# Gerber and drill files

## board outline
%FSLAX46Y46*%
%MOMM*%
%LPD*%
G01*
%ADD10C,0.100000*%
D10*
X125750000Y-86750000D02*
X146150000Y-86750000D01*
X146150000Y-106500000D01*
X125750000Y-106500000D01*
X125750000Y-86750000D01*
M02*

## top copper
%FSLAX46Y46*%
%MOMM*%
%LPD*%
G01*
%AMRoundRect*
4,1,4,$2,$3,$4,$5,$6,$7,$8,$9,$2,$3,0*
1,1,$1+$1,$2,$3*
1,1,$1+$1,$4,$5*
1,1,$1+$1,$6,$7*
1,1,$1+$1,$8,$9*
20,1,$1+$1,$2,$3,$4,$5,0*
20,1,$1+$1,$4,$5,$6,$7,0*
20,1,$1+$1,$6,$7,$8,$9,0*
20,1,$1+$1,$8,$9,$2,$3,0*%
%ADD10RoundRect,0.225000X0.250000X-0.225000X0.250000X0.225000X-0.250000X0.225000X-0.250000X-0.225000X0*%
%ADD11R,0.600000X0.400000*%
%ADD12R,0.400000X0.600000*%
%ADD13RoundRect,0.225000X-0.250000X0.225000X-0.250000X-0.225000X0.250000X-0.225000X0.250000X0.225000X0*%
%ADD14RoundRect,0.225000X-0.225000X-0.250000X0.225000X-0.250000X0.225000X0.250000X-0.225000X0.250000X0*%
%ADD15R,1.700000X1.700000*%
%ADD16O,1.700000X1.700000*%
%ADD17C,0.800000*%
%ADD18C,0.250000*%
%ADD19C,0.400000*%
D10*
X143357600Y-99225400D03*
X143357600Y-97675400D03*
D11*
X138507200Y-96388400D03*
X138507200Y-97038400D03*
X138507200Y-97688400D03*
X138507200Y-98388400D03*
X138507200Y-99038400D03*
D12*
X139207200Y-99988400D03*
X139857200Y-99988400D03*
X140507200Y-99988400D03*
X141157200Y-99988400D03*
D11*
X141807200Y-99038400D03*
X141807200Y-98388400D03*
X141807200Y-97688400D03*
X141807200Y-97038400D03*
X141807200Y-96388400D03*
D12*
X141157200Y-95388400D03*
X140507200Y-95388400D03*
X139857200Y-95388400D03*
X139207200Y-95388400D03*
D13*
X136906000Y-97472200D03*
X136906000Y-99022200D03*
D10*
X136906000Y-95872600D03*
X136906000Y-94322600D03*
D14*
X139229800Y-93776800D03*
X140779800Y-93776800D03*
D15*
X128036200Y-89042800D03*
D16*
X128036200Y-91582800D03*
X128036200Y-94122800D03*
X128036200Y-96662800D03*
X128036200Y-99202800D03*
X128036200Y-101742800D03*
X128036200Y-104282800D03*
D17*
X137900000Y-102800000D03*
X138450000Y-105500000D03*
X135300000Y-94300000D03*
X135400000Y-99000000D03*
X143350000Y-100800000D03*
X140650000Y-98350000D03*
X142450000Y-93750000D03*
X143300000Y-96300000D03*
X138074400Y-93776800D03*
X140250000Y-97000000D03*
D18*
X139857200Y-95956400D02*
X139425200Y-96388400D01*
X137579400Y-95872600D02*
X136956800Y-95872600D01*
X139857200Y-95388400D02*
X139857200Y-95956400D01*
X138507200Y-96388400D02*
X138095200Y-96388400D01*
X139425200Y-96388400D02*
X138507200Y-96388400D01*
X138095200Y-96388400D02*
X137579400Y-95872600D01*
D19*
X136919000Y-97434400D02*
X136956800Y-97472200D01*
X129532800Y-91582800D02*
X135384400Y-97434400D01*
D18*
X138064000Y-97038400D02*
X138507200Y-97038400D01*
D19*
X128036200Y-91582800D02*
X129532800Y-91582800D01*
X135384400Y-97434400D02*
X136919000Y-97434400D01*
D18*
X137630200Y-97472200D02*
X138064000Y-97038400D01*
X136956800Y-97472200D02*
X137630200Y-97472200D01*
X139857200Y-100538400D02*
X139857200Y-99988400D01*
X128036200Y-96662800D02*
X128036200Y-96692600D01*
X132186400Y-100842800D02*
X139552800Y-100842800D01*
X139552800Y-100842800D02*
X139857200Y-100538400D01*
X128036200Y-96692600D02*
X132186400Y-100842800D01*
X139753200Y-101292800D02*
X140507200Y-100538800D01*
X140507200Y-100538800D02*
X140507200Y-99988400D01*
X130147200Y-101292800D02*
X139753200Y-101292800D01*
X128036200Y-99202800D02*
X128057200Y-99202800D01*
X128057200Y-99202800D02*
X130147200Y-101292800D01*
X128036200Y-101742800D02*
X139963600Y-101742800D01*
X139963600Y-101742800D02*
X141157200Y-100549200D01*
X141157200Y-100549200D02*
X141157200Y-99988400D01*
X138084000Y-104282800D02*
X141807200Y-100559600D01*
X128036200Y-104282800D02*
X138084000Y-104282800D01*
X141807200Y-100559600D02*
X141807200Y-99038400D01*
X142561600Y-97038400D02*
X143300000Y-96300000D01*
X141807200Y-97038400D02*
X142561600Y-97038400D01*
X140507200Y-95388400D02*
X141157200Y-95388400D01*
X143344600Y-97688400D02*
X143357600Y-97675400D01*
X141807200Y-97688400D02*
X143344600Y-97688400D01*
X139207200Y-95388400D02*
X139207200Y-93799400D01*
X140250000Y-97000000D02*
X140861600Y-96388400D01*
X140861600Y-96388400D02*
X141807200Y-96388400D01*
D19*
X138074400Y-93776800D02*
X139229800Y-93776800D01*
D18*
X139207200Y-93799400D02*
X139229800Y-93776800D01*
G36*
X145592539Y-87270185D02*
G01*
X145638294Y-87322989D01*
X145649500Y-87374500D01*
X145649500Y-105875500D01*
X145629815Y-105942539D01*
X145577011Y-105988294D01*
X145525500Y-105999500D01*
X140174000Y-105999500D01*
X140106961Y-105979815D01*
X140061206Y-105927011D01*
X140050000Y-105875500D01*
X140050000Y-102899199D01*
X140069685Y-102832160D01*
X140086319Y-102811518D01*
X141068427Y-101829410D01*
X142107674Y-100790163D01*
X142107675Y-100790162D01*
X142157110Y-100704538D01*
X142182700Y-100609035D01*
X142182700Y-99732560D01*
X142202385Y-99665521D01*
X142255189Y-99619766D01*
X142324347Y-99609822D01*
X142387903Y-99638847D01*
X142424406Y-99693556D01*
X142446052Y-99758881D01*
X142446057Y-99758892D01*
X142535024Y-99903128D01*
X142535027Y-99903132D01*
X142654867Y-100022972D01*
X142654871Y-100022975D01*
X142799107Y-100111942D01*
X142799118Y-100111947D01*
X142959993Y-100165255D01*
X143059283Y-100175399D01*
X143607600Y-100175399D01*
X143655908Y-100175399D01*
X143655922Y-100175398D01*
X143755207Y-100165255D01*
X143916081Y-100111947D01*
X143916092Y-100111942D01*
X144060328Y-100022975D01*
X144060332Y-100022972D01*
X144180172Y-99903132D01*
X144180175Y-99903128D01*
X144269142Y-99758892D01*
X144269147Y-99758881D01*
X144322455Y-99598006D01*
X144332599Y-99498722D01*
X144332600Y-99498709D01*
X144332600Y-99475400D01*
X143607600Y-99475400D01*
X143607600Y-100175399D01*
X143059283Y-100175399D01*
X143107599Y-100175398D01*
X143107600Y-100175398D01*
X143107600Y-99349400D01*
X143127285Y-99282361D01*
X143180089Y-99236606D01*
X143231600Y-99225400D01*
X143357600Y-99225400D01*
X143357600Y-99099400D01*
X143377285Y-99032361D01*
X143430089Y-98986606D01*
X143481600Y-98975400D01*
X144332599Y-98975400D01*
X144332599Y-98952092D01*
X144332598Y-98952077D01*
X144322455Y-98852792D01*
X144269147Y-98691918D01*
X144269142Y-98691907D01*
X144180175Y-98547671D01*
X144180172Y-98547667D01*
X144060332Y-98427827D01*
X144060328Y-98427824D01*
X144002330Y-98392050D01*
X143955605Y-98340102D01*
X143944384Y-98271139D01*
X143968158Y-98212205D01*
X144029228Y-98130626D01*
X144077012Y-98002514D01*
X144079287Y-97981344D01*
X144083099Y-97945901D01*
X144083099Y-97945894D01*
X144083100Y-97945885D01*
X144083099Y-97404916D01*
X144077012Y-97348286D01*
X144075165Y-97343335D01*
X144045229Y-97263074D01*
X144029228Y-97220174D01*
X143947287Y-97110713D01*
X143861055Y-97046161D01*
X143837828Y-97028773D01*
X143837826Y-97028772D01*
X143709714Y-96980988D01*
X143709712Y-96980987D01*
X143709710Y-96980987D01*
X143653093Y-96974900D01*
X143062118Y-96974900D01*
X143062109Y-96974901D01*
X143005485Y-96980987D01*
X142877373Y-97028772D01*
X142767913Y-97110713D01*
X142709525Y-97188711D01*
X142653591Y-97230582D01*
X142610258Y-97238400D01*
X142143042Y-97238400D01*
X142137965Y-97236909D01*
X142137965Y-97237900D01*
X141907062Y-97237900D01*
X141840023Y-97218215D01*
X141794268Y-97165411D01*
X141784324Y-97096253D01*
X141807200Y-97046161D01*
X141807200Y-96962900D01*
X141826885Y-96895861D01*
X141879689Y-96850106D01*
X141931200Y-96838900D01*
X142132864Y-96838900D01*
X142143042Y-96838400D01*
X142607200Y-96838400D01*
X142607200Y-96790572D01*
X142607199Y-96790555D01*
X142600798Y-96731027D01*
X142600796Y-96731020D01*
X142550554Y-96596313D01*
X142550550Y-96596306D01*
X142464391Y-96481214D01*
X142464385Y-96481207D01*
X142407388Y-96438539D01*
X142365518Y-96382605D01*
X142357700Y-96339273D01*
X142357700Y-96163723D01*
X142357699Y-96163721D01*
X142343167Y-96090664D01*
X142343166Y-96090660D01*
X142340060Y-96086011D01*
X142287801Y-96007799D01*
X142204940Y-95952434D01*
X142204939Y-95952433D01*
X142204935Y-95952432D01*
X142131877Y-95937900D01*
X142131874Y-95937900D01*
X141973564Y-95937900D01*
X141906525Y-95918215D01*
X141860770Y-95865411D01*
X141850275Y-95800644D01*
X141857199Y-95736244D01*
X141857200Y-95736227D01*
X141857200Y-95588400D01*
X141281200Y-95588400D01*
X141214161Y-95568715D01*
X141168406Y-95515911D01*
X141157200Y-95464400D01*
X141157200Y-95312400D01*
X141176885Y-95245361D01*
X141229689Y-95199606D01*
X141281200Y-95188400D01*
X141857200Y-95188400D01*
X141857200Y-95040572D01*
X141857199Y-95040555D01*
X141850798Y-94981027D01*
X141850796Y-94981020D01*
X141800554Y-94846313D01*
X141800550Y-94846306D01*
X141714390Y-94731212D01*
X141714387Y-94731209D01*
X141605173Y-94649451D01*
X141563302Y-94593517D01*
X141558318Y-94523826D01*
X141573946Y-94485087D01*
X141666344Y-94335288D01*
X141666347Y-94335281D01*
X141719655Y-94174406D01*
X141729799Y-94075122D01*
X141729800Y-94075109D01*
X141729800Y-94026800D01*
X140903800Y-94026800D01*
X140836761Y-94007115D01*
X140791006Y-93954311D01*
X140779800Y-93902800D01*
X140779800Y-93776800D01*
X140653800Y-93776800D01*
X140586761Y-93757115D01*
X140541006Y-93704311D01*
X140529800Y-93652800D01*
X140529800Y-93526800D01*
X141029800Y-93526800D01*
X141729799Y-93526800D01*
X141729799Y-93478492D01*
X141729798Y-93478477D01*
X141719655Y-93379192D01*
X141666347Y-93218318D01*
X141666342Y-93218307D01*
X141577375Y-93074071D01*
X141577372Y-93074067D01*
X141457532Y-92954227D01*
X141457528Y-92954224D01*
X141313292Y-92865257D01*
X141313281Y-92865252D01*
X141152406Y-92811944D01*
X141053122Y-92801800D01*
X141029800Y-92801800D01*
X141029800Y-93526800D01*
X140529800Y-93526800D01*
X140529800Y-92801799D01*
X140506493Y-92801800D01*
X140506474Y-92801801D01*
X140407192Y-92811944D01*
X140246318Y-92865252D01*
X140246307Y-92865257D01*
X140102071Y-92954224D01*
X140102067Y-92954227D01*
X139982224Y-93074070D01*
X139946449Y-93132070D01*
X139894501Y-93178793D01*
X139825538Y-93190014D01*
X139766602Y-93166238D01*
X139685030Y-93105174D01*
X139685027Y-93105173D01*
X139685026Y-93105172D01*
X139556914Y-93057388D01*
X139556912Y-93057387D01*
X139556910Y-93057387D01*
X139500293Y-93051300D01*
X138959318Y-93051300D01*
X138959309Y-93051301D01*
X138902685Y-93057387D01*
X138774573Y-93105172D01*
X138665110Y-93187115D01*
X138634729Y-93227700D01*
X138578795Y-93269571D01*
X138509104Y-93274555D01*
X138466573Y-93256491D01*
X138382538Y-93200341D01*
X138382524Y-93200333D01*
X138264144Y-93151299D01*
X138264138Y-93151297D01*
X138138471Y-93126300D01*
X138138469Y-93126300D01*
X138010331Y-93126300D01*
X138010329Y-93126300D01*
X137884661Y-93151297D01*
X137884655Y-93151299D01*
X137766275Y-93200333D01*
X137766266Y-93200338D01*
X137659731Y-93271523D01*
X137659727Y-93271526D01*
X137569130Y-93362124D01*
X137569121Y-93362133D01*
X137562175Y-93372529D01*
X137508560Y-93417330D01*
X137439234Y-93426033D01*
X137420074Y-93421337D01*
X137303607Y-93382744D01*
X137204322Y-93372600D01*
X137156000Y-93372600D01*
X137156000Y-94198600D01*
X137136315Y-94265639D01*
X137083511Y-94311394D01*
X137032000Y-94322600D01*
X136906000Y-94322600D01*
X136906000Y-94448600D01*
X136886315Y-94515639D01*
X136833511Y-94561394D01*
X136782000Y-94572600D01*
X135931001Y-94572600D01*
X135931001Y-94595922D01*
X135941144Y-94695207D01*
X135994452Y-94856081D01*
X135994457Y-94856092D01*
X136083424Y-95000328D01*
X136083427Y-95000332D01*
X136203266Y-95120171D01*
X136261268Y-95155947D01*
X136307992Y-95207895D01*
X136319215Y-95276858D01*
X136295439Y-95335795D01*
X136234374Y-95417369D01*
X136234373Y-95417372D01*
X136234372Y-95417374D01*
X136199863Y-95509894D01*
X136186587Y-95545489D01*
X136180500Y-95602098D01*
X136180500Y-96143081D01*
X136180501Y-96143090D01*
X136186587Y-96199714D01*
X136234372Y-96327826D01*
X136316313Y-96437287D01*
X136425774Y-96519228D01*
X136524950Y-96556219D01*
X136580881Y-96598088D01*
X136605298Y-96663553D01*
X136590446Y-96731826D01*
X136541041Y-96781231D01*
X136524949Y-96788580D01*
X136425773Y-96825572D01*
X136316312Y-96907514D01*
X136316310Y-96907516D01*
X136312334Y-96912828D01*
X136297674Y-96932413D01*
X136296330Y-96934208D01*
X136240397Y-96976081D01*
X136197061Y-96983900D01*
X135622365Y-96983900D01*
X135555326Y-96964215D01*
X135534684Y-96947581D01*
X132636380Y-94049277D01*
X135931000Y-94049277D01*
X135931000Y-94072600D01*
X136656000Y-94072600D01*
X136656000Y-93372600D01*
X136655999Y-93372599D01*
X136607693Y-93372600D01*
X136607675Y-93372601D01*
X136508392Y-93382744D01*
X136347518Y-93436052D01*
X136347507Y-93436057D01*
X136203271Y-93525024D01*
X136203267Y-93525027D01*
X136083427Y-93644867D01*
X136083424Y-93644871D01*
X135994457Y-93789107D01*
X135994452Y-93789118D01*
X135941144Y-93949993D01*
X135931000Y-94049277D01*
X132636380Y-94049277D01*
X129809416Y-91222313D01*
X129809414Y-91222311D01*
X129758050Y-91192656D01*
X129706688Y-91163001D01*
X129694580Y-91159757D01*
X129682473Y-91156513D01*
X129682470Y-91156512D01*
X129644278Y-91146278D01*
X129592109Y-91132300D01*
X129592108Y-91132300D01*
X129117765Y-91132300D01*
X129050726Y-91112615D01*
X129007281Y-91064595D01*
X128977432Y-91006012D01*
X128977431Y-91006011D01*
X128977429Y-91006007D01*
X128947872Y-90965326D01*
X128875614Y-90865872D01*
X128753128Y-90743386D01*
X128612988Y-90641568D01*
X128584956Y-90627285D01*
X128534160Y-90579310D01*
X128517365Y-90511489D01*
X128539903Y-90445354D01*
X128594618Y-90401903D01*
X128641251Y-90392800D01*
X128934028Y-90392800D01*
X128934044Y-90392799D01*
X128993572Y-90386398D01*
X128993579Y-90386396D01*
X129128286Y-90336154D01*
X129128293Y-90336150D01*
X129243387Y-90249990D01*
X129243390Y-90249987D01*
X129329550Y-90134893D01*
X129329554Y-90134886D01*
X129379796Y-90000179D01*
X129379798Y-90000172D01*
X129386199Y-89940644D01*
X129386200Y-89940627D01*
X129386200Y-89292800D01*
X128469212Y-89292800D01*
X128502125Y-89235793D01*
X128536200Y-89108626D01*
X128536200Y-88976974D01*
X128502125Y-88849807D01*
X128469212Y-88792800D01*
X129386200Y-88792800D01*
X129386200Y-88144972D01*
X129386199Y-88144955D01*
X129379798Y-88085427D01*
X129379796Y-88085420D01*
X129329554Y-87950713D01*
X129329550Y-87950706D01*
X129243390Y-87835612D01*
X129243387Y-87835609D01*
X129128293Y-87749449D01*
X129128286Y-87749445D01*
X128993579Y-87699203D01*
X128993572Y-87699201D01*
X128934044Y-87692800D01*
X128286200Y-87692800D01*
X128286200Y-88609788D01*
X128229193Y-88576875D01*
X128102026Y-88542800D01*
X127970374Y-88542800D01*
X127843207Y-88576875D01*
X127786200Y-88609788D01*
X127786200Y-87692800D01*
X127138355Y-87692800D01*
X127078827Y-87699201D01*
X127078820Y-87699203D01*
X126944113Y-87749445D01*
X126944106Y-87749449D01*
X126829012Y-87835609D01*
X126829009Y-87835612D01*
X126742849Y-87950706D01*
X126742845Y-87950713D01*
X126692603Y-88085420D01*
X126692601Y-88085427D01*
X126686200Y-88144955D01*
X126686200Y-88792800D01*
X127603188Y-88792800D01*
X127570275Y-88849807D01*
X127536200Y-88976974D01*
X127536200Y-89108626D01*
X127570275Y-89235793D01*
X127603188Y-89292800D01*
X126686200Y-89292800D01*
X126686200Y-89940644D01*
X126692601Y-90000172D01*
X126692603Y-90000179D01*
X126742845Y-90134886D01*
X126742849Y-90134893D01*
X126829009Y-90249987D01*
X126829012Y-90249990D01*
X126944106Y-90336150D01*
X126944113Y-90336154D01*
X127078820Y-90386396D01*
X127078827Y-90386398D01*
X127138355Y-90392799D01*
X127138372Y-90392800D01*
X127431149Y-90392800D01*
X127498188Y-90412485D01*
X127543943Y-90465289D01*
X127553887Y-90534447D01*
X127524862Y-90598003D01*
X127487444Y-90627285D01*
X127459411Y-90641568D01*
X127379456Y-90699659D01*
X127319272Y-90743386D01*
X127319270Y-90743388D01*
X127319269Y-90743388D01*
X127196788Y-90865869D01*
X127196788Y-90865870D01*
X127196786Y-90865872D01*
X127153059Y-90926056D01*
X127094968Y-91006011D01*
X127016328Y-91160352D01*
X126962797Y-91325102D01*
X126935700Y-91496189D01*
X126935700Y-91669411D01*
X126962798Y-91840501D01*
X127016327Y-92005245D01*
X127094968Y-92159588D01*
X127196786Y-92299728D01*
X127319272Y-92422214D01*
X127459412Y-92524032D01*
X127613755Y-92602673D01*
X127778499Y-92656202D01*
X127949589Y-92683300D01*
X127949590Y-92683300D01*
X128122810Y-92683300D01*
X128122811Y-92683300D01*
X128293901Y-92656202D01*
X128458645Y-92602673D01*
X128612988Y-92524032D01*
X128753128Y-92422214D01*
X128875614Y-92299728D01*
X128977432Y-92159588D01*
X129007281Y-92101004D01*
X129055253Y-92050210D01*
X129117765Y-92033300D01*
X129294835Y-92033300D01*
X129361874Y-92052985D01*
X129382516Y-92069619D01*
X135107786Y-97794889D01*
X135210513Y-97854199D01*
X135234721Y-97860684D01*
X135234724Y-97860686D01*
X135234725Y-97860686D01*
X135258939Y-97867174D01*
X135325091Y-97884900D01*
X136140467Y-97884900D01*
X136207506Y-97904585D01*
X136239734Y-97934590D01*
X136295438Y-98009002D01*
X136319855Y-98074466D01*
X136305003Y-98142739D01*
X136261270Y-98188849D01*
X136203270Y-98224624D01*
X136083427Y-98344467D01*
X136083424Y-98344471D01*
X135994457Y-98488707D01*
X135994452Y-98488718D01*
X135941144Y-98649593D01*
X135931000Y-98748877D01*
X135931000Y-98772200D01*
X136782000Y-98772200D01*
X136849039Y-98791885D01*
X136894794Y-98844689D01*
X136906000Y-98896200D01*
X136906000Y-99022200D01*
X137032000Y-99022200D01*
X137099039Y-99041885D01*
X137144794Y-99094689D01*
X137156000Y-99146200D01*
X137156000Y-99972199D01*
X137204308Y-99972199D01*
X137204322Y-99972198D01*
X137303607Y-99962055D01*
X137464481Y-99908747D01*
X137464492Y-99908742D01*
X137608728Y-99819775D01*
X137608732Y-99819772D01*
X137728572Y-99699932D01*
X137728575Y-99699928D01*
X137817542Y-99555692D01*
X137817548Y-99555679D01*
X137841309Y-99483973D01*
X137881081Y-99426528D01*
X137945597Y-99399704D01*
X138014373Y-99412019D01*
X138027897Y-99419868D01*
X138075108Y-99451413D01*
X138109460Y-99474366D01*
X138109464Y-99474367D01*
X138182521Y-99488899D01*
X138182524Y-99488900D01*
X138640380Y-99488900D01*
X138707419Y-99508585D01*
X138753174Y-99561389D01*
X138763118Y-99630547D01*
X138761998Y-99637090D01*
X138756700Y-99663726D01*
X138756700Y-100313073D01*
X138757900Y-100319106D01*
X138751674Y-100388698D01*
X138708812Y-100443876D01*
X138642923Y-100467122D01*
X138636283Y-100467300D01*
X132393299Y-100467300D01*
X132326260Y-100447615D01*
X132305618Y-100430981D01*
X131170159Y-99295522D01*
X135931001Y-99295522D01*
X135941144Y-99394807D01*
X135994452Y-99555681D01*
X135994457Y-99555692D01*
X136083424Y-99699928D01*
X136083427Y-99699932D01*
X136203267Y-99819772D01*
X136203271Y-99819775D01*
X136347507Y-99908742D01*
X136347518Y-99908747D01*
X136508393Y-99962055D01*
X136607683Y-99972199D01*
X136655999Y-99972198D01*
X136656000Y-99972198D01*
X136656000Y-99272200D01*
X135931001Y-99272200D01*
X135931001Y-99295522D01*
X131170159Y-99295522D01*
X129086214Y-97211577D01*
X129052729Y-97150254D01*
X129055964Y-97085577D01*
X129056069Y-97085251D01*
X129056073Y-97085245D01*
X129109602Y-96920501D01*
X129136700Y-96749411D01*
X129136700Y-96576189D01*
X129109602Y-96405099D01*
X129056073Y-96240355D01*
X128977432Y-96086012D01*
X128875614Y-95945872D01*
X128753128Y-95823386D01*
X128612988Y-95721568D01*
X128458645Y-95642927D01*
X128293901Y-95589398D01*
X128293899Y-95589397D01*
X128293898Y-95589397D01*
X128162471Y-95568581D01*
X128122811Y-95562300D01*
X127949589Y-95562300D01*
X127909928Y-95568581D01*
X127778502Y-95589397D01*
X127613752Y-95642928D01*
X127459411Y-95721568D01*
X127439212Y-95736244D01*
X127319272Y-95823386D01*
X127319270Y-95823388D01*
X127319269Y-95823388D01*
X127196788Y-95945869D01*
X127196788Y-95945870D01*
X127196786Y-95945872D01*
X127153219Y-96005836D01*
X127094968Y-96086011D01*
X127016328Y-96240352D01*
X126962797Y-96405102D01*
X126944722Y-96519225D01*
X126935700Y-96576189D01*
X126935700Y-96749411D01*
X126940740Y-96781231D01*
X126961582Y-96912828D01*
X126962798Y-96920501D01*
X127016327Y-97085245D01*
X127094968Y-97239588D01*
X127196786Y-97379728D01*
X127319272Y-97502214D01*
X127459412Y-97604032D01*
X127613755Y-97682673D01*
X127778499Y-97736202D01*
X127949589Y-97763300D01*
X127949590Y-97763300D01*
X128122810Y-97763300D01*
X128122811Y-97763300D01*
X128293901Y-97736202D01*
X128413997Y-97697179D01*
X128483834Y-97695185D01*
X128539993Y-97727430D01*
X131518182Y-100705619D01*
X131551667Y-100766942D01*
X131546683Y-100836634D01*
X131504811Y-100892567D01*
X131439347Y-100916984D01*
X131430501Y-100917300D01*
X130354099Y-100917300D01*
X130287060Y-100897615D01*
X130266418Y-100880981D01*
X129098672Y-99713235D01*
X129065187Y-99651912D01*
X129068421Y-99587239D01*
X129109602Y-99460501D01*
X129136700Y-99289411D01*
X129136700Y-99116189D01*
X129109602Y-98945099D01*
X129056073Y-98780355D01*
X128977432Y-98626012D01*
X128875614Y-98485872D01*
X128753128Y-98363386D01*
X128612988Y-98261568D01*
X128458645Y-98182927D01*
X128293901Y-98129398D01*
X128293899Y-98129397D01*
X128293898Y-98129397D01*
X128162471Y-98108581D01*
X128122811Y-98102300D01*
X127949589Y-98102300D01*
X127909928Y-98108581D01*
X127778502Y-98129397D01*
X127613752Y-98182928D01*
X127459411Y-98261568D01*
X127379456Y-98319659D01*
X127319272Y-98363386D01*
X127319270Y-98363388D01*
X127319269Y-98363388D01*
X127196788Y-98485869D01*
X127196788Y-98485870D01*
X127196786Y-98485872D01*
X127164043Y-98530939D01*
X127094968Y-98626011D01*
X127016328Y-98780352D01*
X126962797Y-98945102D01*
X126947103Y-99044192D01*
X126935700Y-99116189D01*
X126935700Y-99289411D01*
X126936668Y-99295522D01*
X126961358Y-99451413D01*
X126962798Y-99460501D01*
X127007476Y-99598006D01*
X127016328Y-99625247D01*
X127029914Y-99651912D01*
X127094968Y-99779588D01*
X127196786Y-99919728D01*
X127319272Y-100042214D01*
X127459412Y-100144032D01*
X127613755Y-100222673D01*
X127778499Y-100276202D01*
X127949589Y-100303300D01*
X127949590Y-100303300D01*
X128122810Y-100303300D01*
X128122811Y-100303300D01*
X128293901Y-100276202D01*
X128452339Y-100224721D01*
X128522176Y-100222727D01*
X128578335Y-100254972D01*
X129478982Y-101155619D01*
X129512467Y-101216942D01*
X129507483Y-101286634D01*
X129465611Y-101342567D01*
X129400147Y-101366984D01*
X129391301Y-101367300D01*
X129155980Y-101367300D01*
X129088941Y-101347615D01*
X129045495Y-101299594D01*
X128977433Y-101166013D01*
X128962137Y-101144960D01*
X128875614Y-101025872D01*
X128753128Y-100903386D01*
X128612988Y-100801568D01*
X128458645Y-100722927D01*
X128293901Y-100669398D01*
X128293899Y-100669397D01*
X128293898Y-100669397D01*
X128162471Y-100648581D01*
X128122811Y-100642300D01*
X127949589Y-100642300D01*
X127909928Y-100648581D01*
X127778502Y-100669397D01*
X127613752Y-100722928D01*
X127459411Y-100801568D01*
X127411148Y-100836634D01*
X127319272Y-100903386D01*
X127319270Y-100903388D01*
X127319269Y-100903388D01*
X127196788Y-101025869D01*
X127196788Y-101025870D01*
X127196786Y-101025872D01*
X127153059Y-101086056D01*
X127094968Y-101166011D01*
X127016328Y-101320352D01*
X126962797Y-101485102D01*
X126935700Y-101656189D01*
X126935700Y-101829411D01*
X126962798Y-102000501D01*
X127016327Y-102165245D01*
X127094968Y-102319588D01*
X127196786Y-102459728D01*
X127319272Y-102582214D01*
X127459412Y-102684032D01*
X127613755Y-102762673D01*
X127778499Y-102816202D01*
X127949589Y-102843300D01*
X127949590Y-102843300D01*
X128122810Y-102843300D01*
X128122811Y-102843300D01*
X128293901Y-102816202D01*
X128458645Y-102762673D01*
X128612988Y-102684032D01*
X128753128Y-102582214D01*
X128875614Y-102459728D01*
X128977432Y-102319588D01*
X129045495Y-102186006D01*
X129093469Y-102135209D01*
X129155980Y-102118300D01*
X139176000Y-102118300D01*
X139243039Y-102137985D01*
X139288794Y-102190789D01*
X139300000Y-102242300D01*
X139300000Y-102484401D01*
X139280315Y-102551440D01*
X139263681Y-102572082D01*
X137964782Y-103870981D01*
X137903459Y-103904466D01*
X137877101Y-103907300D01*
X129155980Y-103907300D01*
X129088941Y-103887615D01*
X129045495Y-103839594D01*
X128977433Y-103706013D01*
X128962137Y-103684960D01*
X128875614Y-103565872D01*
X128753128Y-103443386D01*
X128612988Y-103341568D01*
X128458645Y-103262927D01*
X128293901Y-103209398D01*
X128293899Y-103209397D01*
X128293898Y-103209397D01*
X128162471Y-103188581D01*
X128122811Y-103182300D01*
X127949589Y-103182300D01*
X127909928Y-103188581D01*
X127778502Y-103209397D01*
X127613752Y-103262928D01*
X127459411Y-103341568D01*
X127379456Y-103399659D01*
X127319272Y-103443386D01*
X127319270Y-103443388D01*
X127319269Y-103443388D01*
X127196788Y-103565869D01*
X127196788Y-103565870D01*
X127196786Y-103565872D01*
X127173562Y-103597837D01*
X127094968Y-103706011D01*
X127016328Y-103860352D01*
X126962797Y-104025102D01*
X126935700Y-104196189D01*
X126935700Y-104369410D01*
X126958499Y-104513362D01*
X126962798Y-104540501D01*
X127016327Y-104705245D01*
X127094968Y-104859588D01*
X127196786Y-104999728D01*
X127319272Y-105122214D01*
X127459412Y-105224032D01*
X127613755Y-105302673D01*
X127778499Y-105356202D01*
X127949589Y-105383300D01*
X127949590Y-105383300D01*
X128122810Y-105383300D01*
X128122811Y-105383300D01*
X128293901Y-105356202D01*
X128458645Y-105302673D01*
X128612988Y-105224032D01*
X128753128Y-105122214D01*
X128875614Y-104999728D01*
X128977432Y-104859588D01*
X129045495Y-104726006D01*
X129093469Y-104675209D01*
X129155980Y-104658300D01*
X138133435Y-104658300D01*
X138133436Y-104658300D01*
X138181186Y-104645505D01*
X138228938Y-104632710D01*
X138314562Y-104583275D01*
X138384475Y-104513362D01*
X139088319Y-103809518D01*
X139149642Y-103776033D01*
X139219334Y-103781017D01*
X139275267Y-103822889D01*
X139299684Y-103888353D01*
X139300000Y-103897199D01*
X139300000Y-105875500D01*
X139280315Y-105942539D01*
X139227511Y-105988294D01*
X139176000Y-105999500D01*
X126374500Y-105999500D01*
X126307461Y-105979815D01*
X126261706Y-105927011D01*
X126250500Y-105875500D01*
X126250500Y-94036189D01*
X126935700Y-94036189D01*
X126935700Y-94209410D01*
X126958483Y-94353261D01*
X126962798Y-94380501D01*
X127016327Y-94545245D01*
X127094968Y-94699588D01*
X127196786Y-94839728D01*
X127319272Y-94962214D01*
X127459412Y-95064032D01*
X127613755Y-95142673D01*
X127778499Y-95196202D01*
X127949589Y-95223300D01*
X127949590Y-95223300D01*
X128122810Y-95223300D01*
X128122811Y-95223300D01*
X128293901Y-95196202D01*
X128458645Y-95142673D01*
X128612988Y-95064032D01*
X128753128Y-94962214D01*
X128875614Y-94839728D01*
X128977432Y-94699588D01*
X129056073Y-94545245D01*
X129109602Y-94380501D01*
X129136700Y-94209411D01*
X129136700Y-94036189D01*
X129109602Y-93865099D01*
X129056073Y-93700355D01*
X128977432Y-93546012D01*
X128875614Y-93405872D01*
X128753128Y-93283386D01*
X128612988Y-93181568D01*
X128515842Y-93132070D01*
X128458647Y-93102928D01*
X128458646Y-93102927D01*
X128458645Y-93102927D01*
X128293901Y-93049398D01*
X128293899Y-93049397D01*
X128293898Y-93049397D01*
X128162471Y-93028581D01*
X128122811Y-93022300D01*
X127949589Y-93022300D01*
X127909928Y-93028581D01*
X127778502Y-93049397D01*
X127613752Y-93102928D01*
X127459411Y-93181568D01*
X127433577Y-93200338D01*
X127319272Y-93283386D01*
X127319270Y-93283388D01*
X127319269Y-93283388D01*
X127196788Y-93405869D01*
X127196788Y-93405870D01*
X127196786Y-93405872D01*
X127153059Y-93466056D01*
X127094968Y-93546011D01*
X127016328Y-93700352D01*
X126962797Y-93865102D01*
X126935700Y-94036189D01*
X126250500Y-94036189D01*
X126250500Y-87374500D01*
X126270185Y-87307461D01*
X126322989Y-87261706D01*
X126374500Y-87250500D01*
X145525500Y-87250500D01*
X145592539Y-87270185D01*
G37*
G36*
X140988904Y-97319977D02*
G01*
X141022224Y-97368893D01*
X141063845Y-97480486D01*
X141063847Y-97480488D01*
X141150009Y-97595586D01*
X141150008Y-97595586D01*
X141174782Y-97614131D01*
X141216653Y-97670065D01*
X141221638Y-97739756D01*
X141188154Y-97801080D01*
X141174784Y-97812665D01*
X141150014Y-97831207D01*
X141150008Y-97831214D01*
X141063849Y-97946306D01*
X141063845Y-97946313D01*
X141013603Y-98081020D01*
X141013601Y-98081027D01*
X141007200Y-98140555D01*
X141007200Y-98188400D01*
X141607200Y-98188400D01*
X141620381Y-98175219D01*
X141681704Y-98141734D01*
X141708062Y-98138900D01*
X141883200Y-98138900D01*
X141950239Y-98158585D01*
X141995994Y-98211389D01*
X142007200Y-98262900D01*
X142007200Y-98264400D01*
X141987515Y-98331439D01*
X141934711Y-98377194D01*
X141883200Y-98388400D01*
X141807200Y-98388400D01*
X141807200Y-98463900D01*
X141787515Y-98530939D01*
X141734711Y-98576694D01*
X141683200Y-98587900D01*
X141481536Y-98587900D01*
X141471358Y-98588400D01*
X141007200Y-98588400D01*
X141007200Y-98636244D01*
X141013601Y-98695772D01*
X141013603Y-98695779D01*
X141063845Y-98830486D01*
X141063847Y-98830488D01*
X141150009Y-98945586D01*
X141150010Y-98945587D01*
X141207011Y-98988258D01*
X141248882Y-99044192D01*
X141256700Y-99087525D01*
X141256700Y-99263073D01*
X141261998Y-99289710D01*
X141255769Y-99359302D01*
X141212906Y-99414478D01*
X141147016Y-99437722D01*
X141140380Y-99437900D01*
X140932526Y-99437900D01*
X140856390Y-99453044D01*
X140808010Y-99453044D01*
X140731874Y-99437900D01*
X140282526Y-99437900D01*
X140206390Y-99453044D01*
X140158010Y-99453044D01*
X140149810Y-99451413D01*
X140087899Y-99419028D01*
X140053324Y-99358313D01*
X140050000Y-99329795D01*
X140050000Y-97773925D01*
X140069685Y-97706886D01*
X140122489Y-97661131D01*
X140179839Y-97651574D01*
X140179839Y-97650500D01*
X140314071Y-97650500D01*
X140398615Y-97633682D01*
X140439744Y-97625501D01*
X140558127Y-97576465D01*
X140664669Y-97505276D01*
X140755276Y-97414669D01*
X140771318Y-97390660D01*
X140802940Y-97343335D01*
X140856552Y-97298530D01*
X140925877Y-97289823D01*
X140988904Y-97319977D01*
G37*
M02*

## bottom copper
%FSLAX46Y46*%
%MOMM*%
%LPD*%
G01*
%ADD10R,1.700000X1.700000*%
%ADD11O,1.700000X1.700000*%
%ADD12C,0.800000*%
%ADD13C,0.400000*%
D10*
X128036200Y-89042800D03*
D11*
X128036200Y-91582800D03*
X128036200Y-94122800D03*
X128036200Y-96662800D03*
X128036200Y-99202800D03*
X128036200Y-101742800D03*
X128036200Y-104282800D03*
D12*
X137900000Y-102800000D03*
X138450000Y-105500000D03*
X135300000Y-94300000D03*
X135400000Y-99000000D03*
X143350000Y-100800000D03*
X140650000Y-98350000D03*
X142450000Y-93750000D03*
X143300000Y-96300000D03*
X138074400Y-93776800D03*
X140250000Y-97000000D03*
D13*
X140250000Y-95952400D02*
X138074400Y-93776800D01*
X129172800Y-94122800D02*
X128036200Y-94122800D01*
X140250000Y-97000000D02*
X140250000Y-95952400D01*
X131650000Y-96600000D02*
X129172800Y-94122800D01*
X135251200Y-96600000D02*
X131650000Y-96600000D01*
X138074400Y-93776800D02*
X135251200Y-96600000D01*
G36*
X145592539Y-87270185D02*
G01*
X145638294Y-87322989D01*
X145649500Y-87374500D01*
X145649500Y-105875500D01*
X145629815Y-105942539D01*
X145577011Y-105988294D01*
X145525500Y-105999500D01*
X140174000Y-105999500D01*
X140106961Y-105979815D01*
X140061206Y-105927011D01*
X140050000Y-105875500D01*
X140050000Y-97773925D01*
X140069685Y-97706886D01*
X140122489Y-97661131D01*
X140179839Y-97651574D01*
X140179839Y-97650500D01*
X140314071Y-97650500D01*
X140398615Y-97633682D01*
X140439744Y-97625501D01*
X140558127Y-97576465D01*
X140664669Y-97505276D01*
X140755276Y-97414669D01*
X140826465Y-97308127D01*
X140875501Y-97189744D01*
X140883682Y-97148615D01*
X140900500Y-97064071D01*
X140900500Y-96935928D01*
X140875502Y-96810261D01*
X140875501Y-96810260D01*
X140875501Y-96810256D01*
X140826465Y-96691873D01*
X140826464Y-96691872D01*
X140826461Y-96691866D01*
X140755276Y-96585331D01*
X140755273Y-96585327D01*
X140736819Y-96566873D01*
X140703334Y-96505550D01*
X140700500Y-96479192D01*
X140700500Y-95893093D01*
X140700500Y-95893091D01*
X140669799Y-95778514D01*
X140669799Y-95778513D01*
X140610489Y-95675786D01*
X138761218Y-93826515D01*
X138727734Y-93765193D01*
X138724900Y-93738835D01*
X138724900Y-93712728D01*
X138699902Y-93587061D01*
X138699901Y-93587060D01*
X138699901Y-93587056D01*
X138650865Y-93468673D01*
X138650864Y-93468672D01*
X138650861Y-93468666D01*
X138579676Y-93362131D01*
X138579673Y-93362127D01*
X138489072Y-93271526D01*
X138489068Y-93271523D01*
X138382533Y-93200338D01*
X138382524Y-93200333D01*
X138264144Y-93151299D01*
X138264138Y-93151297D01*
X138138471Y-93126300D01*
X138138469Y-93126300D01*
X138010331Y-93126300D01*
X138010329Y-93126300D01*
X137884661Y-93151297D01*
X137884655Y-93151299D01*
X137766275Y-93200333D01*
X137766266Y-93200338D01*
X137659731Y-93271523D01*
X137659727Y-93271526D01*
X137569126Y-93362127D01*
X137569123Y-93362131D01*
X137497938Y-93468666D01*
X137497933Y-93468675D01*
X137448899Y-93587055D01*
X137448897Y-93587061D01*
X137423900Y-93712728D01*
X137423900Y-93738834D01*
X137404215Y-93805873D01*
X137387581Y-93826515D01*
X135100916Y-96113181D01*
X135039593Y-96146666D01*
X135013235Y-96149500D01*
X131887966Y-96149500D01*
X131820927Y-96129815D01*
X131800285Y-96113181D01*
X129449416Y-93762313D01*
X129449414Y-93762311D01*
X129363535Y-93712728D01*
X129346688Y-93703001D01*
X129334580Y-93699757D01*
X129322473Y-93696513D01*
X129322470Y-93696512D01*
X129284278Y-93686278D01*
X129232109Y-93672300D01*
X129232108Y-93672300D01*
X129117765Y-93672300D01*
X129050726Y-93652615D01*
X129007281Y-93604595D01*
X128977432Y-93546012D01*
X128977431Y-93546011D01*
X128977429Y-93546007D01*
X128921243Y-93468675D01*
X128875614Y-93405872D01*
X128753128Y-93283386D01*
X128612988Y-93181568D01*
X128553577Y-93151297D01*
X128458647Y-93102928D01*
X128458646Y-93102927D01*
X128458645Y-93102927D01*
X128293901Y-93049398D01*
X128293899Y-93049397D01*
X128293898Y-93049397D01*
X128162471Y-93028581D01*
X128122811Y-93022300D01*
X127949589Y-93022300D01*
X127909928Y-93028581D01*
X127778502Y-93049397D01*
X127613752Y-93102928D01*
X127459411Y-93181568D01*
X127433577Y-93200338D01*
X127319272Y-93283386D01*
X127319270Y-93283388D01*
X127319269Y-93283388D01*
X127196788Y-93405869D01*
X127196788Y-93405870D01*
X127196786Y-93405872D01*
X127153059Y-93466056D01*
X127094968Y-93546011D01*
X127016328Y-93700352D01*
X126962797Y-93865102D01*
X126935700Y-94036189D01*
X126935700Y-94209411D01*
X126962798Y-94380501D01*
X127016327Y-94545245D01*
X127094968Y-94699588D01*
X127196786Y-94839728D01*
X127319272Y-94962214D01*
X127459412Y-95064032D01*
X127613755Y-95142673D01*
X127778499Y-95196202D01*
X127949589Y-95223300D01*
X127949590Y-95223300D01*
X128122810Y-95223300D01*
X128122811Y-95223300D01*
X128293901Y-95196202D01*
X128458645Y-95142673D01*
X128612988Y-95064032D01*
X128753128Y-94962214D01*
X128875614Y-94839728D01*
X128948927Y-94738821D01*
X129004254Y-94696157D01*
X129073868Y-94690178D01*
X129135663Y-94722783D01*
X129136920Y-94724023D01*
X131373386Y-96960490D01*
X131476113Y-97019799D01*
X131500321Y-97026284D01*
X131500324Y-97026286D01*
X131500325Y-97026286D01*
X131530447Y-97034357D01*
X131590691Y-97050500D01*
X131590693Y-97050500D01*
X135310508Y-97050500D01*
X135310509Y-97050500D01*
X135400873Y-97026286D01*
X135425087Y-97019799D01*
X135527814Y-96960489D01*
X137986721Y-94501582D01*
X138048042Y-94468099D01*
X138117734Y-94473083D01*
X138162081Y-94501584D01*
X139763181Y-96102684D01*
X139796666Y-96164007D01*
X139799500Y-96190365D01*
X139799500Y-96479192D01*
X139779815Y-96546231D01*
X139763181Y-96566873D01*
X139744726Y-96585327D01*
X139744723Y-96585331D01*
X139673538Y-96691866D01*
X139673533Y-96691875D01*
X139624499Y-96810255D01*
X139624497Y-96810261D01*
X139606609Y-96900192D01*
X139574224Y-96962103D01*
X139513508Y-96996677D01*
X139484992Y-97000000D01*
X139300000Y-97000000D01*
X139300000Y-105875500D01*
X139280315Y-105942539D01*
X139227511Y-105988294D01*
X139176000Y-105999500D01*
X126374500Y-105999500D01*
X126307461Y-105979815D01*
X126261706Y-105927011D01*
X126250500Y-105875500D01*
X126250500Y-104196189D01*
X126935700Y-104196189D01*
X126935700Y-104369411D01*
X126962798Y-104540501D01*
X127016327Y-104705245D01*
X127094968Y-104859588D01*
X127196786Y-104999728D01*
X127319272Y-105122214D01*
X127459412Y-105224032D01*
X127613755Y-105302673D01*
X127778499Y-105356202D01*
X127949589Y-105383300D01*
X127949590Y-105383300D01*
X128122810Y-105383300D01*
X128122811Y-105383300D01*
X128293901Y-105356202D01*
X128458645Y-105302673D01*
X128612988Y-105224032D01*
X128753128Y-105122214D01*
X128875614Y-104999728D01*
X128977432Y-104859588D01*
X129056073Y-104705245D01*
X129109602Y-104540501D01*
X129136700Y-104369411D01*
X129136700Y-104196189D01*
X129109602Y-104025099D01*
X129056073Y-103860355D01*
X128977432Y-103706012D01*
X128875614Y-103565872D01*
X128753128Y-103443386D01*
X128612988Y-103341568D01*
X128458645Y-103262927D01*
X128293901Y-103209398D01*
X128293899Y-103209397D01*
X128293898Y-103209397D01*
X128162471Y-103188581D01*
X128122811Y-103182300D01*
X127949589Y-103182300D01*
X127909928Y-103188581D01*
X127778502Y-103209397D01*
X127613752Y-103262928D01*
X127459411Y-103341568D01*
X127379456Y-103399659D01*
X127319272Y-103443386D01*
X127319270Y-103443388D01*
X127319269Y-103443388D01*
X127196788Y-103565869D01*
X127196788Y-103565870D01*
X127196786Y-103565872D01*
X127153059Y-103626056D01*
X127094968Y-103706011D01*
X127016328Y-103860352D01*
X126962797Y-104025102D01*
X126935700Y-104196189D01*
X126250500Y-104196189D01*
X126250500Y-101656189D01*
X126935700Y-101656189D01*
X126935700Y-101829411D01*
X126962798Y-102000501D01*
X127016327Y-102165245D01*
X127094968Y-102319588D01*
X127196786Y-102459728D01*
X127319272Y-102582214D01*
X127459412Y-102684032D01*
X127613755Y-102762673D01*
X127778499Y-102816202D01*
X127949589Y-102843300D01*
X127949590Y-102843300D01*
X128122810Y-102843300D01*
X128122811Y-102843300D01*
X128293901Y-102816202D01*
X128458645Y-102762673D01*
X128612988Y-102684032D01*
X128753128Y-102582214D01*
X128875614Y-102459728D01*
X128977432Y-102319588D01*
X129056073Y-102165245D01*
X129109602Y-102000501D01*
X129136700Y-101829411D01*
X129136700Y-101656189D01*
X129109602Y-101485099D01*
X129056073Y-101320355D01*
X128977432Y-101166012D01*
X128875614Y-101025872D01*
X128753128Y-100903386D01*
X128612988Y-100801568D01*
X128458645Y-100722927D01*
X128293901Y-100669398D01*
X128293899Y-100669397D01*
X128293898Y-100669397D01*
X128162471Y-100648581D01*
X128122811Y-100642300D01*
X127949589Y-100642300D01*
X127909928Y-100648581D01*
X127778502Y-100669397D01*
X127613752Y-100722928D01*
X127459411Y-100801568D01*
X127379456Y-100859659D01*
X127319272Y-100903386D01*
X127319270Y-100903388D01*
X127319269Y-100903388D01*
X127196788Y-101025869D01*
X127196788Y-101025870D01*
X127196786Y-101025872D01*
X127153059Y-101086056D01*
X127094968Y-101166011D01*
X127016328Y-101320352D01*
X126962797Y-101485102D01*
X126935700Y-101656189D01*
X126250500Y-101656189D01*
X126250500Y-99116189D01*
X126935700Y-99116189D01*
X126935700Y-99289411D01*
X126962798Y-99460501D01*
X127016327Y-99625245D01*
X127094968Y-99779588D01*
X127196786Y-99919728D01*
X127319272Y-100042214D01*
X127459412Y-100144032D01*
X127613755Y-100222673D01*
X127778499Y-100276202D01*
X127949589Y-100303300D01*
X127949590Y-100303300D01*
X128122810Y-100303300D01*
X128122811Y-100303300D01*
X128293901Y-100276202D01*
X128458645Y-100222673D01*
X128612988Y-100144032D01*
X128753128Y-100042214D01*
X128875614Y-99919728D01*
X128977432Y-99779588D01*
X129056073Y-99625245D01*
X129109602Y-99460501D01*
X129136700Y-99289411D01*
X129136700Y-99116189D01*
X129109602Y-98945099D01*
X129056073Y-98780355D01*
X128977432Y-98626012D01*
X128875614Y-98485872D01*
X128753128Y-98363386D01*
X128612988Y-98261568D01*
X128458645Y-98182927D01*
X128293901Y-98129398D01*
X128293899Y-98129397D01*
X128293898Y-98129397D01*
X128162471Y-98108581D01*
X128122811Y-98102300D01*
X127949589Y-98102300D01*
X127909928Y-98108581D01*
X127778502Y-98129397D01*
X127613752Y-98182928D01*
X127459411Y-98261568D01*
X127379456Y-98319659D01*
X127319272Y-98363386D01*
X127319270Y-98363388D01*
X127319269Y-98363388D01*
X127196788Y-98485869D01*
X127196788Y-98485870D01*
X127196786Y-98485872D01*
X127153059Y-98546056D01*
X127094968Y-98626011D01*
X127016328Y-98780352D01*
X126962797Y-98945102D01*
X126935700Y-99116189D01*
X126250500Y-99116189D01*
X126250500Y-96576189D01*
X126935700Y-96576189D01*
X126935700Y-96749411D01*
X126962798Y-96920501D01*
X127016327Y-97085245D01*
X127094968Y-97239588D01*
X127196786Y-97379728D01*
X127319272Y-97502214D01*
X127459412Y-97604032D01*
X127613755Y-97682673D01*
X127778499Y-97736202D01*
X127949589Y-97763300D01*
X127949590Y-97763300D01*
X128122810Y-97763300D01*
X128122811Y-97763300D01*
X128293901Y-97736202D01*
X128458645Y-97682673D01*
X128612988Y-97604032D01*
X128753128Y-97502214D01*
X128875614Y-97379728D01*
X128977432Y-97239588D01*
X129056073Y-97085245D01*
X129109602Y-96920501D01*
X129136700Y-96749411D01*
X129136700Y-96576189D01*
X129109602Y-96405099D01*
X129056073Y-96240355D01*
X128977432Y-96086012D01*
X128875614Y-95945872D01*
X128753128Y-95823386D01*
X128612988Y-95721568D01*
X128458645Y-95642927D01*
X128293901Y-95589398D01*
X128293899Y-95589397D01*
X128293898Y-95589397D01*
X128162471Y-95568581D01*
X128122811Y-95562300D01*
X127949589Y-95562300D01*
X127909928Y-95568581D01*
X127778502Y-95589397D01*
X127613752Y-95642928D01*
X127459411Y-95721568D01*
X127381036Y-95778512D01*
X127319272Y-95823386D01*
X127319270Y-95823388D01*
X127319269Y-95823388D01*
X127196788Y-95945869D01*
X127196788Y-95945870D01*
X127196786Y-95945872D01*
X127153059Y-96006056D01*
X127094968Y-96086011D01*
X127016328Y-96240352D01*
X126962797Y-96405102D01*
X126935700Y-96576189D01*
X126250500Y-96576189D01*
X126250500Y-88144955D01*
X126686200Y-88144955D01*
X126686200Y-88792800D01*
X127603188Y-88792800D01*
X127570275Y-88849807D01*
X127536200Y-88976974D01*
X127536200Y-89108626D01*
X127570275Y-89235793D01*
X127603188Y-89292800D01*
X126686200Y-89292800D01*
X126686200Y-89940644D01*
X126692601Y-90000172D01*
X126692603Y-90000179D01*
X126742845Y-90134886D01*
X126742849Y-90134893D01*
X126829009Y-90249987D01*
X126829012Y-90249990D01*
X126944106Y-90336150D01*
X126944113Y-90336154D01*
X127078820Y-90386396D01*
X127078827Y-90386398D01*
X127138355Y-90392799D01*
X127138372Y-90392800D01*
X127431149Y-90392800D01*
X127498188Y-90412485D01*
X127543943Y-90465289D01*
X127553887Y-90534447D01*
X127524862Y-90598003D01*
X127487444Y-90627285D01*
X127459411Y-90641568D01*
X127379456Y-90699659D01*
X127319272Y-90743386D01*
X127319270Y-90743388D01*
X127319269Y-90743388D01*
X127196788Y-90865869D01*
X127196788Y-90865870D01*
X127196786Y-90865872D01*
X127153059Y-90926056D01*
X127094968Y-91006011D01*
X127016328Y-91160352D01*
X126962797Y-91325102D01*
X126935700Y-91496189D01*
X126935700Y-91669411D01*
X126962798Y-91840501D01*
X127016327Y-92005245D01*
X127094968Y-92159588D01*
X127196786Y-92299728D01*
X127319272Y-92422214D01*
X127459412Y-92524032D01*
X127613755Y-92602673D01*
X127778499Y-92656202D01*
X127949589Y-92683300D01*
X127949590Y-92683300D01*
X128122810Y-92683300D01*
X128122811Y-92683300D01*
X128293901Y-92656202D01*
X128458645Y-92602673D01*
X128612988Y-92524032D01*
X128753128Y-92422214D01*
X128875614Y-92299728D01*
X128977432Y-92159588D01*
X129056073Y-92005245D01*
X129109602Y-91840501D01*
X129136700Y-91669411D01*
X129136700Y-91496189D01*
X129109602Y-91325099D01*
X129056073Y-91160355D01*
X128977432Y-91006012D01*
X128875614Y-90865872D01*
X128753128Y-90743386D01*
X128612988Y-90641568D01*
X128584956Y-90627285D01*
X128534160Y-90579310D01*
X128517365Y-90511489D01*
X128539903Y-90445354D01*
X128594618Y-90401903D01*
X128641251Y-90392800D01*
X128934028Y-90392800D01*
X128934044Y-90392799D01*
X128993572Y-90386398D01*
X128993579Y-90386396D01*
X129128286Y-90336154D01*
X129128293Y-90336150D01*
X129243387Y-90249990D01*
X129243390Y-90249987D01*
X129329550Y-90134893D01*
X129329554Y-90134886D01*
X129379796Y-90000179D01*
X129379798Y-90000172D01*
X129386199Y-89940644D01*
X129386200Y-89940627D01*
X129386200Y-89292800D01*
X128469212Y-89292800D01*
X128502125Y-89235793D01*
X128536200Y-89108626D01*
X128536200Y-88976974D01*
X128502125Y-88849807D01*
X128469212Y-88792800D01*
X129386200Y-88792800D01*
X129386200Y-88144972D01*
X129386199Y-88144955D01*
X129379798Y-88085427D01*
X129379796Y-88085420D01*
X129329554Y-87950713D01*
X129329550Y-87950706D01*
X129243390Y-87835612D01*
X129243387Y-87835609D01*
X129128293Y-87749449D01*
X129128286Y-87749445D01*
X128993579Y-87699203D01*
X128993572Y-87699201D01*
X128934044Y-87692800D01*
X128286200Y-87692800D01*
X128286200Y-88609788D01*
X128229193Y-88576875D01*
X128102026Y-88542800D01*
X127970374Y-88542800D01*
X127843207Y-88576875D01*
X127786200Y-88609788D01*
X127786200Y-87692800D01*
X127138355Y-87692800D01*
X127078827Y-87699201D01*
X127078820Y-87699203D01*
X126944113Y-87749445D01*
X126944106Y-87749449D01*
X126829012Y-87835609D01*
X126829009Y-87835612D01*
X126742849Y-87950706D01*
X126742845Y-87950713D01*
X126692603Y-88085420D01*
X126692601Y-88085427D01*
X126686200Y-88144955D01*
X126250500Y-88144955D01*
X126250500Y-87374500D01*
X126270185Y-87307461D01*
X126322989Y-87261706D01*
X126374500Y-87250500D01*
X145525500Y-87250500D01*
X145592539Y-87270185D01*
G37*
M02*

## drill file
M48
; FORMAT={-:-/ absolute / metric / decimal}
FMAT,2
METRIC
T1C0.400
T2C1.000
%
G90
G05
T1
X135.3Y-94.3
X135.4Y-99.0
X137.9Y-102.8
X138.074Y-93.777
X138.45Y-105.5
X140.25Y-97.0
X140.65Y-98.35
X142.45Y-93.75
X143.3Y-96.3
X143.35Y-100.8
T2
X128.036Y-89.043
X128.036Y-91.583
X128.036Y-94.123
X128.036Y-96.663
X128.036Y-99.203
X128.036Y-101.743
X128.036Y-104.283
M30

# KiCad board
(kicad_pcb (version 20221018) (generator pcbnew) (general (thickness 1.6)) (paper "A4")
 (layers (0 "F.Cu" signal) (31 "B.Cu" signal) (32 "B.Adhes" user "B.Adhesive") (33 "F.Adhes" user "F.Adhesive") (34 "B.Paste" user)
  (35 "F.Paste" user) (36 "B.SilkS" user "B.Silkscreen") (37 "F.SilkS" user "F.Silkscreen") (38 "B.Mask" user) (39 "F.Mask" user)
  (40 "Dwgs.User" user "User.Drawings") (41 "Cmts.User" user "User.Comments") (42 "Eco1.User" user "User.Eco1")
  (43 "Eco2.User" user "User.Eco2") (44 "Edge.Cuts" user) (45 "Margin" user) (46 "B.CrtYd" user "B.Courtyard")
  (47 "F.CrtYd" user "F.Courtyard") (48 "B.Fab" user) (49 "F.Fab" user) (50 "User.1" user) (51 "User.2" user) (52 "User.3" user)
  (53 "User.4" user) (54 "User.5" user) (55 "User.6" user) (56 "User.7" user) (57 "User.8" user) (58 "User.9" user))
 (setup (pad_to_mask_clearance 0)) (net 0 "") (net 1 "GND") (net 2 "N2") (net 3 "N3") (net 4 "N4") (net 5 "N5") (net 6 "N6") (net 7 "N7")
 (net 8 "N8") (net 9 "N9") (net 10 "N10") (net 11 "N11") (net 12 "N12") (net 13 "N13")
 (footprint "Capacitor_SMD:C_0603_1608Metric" (layer "F.Cu") (at 143.3576 98.4504 90)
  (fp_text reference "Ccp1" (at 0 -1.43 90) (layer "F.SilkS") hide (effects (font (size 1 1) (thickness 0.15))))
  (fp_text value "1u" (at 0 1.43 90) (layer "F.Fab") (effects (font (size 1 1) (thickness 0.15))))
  (pad "1" smd roundrect (at -0.775 0 90) (size 0.9 0.95) (layers "F.Cu" "F.Paste" "F.Mask") (roundrect_rratio 0.25) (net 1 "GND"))
  (pad "2" smd roundrect (at 0.775 0 90) (size 0.9 0.95) (layers "F.Cu" "F.Paste" "F.Mask") (roundrect_rratio 0.25) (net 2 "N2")))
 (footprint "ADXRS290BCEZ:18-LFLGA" (layer "F.Cu") (at 140.1572 97.6884)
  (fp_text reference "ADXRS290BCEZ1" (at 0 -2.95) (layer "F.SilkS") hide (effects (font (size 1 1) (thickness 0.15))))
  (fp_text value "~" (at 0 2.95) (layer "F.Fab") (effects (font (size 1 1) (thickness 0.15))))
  (pad "1" smd rect (at -1.65 -1.3) (size 0.6 0.4) (layers "F.Cu" "F.Paste" "F.Mask") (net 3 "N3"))
  (pad "2" smd rect (at -1.65 -0.65) (size 0.6 0.4) (layers "F.Cu" "F.Paste" "F.Mask") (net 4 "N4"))
  (pad "3" smd rect (at -1.65 0) (size 0.6 0.4) (layers "F.Cu" "F.Paste" "F.Mask") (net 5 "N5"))
  (pad "4" smd rect (at -1.65 0.7) (size 0.6 0.4) (layers "F.Cu" "F.Paste" "F.Mask") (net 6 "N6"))
  (pad "5" smd rect (at -1.65 1.35) (size 0.6 0.4) (layers "F.Cu" "F.Paste" "F.Mask") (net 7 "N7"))
  (pad "6" smd rect (at -0.95 2.3 90) (size 0.6 0.4) (layers "F.Cu" "F.Paste" "F.Mask") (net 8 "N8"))
  (pad "7" smd rect (at -0.3 2.3 90) (size 0.6 0.4) (layers "F.Cu" "F.Paste" "F.Mask") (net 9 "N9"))
  (pad "8" smd rect (at 0.35 2.3 90) (size 0.6 0.4) (layers "F.Cu" "F.Paste" "F.Mask") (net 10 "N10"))
  (pad "9" smd rect (at 1 2.3 90) (size 0.6 0.4) (layers "F.Cu" "F.Paste" "F.Mask") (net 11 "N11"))
  (pad "10" smd rect (at 1.65 1.35 180) (size 0.6 0.4) (layers "F.Cu" "F.Paste" "F.Mask") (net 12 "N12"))
  (pad "11" smd rect (at 1.65 0.7 180) (size 0.6 0.4) (layers "F.Cu" "F.Paste" "F.Mask") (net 1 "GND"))
  (pad "12" smd rect (at 1.65 0 180) (size 0.6 0.4) (layers "F.Cu" "F.Paste" "F.Mask") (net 2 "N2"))
  (pad "13" smd rect (at 1.65 -0.65 180) (size 0.6 0.4) (layers "F.Cu" "F.Paste" "F.Mask") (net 1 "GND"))
  (pad "14" smd rect (at 1.65 -1.3 180) (size 0.6 0.4) (layers "F.Cu" "F.Paste" "F.Mask") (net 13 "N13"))
  (pad "15" smd rect (at 1 -2.3 90) (size 0.6 0.4) (layers "F.Cu" "F.Paste" "F.Mask") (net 1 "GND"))
  (pad "16" smd rect (at 0.35 -2.3 90) (size 0.6 0.4) (layers "F.Cu" "F.Paste" "F.Mask") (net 1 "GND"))
  (pad "17" smd rect (at -0.3 -2.3 90) (size 0.6 0.4) (layers "F.Cu" "F.Paste" "F.Mask") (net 3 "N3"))
  (pad "18" smd rect (at -0.95 -2.3 90) (size 0.6 0.4) (layers "F.Cu" "F.Paste" "F.Mask") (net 13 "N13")))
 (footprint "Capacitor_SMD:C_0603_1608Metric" (layer "F.Cu") (at 136.906 98.2472 -90)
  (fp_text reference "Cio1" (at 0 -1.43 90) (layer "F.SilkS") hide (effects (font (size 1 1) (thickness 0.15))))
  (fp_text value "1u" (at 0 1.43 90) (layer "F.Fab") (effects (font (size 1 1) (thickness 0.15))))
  (pad "1" smd roundrect (at -0.775 0 270) (size 0.9 0.95) (layers "F.Cu" "F.Paste" "F.Mask") (roundrect_rratio 0.25) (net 4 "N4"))
  (pad "2" smd roundrect (at 0.775 0 270) (size 0.9 0.95) (layers "F.Cu" "F.Paste" "F.Mask") (roundrect_rratio 0.25) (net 1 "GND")))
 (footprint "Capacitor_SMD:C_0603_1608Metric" (layer "F.Cu") (at 136.906 95.0976 90)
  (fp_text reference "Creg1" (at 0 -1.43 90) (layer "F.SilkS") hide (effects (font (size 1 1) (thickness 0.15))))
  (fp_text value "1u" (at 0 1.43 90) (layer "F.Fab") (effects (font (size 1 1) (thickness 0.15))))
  (pad "1" smd roundrect (at -0.775 0 90) (size 0.9 0.95) (layers "F.Cu" "F.Paste" "F.Mask") (roundrect_rratio 0.25) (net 3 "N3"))
  (pad "2" smd roundrect (at 0.775 0 90) (size 0.9 0.95) (layers "F.Cu" "F.Paste" "F.Mask") (roundrect_rratio 0.25) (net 1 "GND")))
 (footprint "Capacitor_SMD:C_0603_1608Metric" (layer "F.Cu") (at 140.0048 93.7768)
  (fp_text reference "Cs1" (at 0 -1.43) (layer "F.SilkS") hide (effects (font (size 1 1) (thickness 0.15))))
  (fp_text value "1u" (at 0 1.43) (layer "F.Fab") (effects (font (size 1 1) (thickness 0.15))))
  (pad "1" smd roundrect (at -0.775 0) (size 0.9 0.95) (layers "F.Cu" "F.Paste" "F.Mask") (roundrect_rratio 0.25) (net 13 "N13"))
  (pad "2" smd roundrect (at 0.775 0) (size 0.9 0.95) (layers "F.Cu" "F.Paste" "F.Mask") (roundrect_rratio 0.25) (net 1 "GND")))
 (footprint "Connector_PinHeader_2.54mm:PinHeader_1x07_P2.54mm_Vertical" (layer "F.Cu") (at 128.0362 89.0428)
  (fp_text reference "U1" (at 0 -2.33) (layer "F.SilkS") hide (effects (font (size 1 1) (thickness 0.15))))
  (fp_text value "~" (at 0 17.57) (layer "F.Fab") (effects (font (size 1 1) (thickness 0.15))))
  (pad "1" thru_hole rect (at 0 0) (size 1.7 1.7) (drill 1) (layers "*.Cu" "*.Mask") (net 1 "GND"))
  (pad "2" thru_hole oval (at 0 2.54) (size 1.7 1.7) (drill 1) (layers "*.Cu" "*.Mask") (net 4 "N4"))
  (pad "3" thru_hole oval (at 0 5.08) (size 1.7 1.7) (drill 1) (layers "*.Cu" "*.Mask") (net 13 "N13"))
  (pad "4" thru_hole oval (at 0 7.62) (size 1.7 1.7) (drill 1) (layers "*.Cu" "*.Mask") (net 9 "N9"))
  (pad "5" thru_hole oval (at 0 10.16) (size 1.7 1.7) (drill 1) (layers "*.Cu" "*.Mask") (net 10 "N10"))
  (pad "6" thru_hole oval (at 0 12.7) (size 1.7 1.7) (drill 1) (layers "*.Cu" "*.Mask") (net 11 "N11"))
  (pad "7" thru_hole oval (at 0 15.24) (size 1.7 1.7) (drill 1) (layers "*.Cu" "*.Mask") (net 12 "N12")))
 (gr_rect (start 125.75 86.75) (end 146.15 106.5) (stroke (width 0.1) (type default)) (fill none) (layer "Edge.Cuts"))
 (segment (start 139.8572 95.9564) (end 139.4252 96.3884) (width 0.25) (layer "F.Cu") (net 3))
 (segment (start 137.5794 95.8726) (end 136.9568 95.8726) (width 0.25) (layer "F.Cu") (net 3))
 (segment (start 139.8572 95.3884) (end 139.8572 95.9564) (width 0.25) (layer "F.Cu") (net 3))
 (segment (start 138.5072 96.3884) (end 138.0952 96.3884) (width 0.25) (layer "F.Cu") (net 3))
 (segment (start 139.4252 96.3884) (end 138.5072 96.3884) (width 0.25) (layer "F.Cu") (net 3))
 (segment (start 138.0952 96.3884) (end 137.5794 95.8726) (width 0.25) (layer "F.Cu") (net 3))
 (segment (start 136.919 97.4344) (end 136.9568 97.4722) (width 0.4) (layer "F.Cu") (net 4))
 (segment (start 129.5328 91.5828) (end 135.3844 97.4344) (width 0.4) (layer "F.Cu") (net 4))
 (segment (start 138.064 97.0384) (end 138.5072 97.0384) (width 0.25) (layer "F.Cu") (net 4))
 (segment (start 128.0362 91.5828) (end 129.5328 91.5828) (width 0.4) (layer "F.Cu") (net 4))
 (segment (start 135.3844 97.4344) (end 136.919 97.4344) (width 0.4) (layer "F.Cu") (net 4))
 (segment (start 137.6302 97.4722) (end 138.064 97.0384) (width 0.25) (layer "F.Cu") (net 4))
 (segment (start 136.9568 97.4722) (end 137.6302 97.4722) (width 0.25) (layer "F.Cu") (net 4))
 (segment (start 139.8572 100.5384) (end 139.8572 99.9884) (width 0.25) (layer "F.Cu") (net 9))
 (segment (start 128.0362 96.6628) (end 128.0362 96.6926) (width 0.25) (layer "F.Cu") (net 9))
 (segment (start 132.1864 100.8428) (end 139.5528 100.8428) (width 0.25) (layer "F.Cu") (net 9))
 (segment (start 139.5528 100.8428) (end 139.8572 100.5384) (width 0.25) (layer "F.Cu") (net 9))
 (segment (start 128.0362 96.6926) (end 132.1864 100.8428) (width 0.25) (layer "F.Cu") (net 9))
 (segment (start 139.7532 101.2928) (end 140.5072 100.5388) (width 0.25) (layer "F.Cu") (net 10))
 (segment (start 140.5072 100.5388) (end 140.5072 99.9884) (width 0.25) (layer "F.Cu") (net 10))
 (segment (start 130.1472 101.2928) (end 139.7532 101.2928) (width 0.25) (layer "F.Cu") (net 10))
 (segment (start 128.0362 99.2028) (end 128.0572 99.2028) (width 0.25) (layer "F.Cu") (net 10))
 (segment (start 128.0572 99.2028) (end 130.1472 101.2928) (width 0.25) (layer "F.Cu") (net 10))
 (segment (start 128.0362 101.7428) (end 139.9636 101.7428) (width 0.25) (layer "F.Cu") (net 11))
 (segment (start 139.9636 101.7428) (end 141.1572 100.5492) (width 0.25) (layer "F.Cu") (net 11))
 (segment (start 141.1572 100.5492) (end 141.1572 99.9884) (width 0.25) (layer "F.Cu") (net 11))
 (segment (start 138.084 104.2828) (end 141.8072 100.5596) (width 0.25) (layer "F.Cu") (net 12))
 (segment (start 128.0362 104.2828) (end 138.084 104.2828) (width 0.25) (layer "F.Cu") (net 12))
 (segment (start 141.8072 100.5596) (end 141.8072 99.0384) (width 0.25) (layer "F.Cu") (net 12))
 (segment (start 142.5616 97.0384) (end 143.3 96.3) (width 0.25) (layer "F.Cu") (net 1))
 (segment (start 141.8072 97.0384) (end 142.5616 97.0384) (width 0.25) (layer "F.Cu") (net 1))
 (segment (start 140.5072 95.3884) (end 141.1572 95.3884) (width 0.25) (layer "F.Cu") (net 1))
 (via (at 137.9 102.8) (size 0.8) (drill 0.4) (layers "F.Cu" "B.Cu") (free) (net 1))
 (via (at 138.45 105.5) (size 0.8) (drill 0.4) (layers "F.Cu" "B.Cu") (free) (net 1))
 (via (at 135.3 94.3) (size 0.8) (drill 0.4) (layers "F.Cu" "B.Cu") (free) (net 1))
 (via (at 135.4 99) (size 0.8) (drill 0.4) (layers "F.Cu" "B.Cu") (free) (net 1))
 (via (at 143.35 100.8) (size 0.8) (drill 0.4) (layers "F.Cu" "B.Cu") (free) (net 1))
 (via (at 140.65 98.35) (size 0.8) (drill 0.4) (layers "F.Cu" "B.Cu") (free) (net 1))
 (via (at 142.45 93.75) (size 0.8) (drill 0.4) (layers "F.Cu" "B.Cu") (free) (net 1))
 (via (at 143.3 96.3) (size 0.8) (drill 0.4) (layers "F.Cu" "B.Cu") (free) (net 1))
 (segment (start 143.3446 97.6884) (end 143.3576 97.6754) (width 0.25) (layer "F.Cu") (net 2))
 (segment (start 141.8072 97.6884) (end 143.3446 97.6884) (width 0.25) (layer "F.Cu") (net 2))
 (segment (start 139.2072 95.3884) (end 139.2072 93.7994) (width 0.25) (layer "F.Cu") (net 13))
 (segment (start 140.25 97) (end 140.8616 96.3884) (width 0.25) (layer "F.Cu") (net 13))
 (segment (start 140.8616 96.3884) (end 141.8072 96.3884) (width 0.25) (layer "F.Cu") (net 13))
 (segment (start 138.0744 93.7768) (end 139.2298 93.7768) (width 0.4) (layer "F.Cu") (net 13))
 (segment (start 139.2072 93.7994) (end 139.2298 93.7768) (width 0.25) (layer "F.Cu") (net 13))
 (via (at 138.0744 93.7768) (size 0.8) (drill 0.4) (layers "F.Cu" "B.Cu") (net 13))
 (via (at 140.25 97) (size 0.8) (drill 0.4) (layers "F.Cu" "B.Cu") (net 13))
 (segment (start 140.25 95.9524) (end 138.0744 93.7768) (width 0.4) (layer "B.Cu") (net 13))
 (segment (start 129.1728 94.1228) (end 128.0362 94.1228) (width 0.4) (layer "B.Cu") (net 13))
 (segment (start 140.25 97) (end 140.25 95.9524) (width 0.4) (layer "B.Cu") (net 13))
 (segment (start 131.65 96.6) (end 129.1728 94.1228) (width 0.4) (layer "B.Cu") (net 13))
 (segment (start 135.2512 96.6) (end 131.65 96.6) (width 0.4) (layer "B.Cu") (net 13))
 (segment (start 138.0744 93.7768) (end 135.2512 96.6) (width 0.4) (layer "B.Cu") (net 13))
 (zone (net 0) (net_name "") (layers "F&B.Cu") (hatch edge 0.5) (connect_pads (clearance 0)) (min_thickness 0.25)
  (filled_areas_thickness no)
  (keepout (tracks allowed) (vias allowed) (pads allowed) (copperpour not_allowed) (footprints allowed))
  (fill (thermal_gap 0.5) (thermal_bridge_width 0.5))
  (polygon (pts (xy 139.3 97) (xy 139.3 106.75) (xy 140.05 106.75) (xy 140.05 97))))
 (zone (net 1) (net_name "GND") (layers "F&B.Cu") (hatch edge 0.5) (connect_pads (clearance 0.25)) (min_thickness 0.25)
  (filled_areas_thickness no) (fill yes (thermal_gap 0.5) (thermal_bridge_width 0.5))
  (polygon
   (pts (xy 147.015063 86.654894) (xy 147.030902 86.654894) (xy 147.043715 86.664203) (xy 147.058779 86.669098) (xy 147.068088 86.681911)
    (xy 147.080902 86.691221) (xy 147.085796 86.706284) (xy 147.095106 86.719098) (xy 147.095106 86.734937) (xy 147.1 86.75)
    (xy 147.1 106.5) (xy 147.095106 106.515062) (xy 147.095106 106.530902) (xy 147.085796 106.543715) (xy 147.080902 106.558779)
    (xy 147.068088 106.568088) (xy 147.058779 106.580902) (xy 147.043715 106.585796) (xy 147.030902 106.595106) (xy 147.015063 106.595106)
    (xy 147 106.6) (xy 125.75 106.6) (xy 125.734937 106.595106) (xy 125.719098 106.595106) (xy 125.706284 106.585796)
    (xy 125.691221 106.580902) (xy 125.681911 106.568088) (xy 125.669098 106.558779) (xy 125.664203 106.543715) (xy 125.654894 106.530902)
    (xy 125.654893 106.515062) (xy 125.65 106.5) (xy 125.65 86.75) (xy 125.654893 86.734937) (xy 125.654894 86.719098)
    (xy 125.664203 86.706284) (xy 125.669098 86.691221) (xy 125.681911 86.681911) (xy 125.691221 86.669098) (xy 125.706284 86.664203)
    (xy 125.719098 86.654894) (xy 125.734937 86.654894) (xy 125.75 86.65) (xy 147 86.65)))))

